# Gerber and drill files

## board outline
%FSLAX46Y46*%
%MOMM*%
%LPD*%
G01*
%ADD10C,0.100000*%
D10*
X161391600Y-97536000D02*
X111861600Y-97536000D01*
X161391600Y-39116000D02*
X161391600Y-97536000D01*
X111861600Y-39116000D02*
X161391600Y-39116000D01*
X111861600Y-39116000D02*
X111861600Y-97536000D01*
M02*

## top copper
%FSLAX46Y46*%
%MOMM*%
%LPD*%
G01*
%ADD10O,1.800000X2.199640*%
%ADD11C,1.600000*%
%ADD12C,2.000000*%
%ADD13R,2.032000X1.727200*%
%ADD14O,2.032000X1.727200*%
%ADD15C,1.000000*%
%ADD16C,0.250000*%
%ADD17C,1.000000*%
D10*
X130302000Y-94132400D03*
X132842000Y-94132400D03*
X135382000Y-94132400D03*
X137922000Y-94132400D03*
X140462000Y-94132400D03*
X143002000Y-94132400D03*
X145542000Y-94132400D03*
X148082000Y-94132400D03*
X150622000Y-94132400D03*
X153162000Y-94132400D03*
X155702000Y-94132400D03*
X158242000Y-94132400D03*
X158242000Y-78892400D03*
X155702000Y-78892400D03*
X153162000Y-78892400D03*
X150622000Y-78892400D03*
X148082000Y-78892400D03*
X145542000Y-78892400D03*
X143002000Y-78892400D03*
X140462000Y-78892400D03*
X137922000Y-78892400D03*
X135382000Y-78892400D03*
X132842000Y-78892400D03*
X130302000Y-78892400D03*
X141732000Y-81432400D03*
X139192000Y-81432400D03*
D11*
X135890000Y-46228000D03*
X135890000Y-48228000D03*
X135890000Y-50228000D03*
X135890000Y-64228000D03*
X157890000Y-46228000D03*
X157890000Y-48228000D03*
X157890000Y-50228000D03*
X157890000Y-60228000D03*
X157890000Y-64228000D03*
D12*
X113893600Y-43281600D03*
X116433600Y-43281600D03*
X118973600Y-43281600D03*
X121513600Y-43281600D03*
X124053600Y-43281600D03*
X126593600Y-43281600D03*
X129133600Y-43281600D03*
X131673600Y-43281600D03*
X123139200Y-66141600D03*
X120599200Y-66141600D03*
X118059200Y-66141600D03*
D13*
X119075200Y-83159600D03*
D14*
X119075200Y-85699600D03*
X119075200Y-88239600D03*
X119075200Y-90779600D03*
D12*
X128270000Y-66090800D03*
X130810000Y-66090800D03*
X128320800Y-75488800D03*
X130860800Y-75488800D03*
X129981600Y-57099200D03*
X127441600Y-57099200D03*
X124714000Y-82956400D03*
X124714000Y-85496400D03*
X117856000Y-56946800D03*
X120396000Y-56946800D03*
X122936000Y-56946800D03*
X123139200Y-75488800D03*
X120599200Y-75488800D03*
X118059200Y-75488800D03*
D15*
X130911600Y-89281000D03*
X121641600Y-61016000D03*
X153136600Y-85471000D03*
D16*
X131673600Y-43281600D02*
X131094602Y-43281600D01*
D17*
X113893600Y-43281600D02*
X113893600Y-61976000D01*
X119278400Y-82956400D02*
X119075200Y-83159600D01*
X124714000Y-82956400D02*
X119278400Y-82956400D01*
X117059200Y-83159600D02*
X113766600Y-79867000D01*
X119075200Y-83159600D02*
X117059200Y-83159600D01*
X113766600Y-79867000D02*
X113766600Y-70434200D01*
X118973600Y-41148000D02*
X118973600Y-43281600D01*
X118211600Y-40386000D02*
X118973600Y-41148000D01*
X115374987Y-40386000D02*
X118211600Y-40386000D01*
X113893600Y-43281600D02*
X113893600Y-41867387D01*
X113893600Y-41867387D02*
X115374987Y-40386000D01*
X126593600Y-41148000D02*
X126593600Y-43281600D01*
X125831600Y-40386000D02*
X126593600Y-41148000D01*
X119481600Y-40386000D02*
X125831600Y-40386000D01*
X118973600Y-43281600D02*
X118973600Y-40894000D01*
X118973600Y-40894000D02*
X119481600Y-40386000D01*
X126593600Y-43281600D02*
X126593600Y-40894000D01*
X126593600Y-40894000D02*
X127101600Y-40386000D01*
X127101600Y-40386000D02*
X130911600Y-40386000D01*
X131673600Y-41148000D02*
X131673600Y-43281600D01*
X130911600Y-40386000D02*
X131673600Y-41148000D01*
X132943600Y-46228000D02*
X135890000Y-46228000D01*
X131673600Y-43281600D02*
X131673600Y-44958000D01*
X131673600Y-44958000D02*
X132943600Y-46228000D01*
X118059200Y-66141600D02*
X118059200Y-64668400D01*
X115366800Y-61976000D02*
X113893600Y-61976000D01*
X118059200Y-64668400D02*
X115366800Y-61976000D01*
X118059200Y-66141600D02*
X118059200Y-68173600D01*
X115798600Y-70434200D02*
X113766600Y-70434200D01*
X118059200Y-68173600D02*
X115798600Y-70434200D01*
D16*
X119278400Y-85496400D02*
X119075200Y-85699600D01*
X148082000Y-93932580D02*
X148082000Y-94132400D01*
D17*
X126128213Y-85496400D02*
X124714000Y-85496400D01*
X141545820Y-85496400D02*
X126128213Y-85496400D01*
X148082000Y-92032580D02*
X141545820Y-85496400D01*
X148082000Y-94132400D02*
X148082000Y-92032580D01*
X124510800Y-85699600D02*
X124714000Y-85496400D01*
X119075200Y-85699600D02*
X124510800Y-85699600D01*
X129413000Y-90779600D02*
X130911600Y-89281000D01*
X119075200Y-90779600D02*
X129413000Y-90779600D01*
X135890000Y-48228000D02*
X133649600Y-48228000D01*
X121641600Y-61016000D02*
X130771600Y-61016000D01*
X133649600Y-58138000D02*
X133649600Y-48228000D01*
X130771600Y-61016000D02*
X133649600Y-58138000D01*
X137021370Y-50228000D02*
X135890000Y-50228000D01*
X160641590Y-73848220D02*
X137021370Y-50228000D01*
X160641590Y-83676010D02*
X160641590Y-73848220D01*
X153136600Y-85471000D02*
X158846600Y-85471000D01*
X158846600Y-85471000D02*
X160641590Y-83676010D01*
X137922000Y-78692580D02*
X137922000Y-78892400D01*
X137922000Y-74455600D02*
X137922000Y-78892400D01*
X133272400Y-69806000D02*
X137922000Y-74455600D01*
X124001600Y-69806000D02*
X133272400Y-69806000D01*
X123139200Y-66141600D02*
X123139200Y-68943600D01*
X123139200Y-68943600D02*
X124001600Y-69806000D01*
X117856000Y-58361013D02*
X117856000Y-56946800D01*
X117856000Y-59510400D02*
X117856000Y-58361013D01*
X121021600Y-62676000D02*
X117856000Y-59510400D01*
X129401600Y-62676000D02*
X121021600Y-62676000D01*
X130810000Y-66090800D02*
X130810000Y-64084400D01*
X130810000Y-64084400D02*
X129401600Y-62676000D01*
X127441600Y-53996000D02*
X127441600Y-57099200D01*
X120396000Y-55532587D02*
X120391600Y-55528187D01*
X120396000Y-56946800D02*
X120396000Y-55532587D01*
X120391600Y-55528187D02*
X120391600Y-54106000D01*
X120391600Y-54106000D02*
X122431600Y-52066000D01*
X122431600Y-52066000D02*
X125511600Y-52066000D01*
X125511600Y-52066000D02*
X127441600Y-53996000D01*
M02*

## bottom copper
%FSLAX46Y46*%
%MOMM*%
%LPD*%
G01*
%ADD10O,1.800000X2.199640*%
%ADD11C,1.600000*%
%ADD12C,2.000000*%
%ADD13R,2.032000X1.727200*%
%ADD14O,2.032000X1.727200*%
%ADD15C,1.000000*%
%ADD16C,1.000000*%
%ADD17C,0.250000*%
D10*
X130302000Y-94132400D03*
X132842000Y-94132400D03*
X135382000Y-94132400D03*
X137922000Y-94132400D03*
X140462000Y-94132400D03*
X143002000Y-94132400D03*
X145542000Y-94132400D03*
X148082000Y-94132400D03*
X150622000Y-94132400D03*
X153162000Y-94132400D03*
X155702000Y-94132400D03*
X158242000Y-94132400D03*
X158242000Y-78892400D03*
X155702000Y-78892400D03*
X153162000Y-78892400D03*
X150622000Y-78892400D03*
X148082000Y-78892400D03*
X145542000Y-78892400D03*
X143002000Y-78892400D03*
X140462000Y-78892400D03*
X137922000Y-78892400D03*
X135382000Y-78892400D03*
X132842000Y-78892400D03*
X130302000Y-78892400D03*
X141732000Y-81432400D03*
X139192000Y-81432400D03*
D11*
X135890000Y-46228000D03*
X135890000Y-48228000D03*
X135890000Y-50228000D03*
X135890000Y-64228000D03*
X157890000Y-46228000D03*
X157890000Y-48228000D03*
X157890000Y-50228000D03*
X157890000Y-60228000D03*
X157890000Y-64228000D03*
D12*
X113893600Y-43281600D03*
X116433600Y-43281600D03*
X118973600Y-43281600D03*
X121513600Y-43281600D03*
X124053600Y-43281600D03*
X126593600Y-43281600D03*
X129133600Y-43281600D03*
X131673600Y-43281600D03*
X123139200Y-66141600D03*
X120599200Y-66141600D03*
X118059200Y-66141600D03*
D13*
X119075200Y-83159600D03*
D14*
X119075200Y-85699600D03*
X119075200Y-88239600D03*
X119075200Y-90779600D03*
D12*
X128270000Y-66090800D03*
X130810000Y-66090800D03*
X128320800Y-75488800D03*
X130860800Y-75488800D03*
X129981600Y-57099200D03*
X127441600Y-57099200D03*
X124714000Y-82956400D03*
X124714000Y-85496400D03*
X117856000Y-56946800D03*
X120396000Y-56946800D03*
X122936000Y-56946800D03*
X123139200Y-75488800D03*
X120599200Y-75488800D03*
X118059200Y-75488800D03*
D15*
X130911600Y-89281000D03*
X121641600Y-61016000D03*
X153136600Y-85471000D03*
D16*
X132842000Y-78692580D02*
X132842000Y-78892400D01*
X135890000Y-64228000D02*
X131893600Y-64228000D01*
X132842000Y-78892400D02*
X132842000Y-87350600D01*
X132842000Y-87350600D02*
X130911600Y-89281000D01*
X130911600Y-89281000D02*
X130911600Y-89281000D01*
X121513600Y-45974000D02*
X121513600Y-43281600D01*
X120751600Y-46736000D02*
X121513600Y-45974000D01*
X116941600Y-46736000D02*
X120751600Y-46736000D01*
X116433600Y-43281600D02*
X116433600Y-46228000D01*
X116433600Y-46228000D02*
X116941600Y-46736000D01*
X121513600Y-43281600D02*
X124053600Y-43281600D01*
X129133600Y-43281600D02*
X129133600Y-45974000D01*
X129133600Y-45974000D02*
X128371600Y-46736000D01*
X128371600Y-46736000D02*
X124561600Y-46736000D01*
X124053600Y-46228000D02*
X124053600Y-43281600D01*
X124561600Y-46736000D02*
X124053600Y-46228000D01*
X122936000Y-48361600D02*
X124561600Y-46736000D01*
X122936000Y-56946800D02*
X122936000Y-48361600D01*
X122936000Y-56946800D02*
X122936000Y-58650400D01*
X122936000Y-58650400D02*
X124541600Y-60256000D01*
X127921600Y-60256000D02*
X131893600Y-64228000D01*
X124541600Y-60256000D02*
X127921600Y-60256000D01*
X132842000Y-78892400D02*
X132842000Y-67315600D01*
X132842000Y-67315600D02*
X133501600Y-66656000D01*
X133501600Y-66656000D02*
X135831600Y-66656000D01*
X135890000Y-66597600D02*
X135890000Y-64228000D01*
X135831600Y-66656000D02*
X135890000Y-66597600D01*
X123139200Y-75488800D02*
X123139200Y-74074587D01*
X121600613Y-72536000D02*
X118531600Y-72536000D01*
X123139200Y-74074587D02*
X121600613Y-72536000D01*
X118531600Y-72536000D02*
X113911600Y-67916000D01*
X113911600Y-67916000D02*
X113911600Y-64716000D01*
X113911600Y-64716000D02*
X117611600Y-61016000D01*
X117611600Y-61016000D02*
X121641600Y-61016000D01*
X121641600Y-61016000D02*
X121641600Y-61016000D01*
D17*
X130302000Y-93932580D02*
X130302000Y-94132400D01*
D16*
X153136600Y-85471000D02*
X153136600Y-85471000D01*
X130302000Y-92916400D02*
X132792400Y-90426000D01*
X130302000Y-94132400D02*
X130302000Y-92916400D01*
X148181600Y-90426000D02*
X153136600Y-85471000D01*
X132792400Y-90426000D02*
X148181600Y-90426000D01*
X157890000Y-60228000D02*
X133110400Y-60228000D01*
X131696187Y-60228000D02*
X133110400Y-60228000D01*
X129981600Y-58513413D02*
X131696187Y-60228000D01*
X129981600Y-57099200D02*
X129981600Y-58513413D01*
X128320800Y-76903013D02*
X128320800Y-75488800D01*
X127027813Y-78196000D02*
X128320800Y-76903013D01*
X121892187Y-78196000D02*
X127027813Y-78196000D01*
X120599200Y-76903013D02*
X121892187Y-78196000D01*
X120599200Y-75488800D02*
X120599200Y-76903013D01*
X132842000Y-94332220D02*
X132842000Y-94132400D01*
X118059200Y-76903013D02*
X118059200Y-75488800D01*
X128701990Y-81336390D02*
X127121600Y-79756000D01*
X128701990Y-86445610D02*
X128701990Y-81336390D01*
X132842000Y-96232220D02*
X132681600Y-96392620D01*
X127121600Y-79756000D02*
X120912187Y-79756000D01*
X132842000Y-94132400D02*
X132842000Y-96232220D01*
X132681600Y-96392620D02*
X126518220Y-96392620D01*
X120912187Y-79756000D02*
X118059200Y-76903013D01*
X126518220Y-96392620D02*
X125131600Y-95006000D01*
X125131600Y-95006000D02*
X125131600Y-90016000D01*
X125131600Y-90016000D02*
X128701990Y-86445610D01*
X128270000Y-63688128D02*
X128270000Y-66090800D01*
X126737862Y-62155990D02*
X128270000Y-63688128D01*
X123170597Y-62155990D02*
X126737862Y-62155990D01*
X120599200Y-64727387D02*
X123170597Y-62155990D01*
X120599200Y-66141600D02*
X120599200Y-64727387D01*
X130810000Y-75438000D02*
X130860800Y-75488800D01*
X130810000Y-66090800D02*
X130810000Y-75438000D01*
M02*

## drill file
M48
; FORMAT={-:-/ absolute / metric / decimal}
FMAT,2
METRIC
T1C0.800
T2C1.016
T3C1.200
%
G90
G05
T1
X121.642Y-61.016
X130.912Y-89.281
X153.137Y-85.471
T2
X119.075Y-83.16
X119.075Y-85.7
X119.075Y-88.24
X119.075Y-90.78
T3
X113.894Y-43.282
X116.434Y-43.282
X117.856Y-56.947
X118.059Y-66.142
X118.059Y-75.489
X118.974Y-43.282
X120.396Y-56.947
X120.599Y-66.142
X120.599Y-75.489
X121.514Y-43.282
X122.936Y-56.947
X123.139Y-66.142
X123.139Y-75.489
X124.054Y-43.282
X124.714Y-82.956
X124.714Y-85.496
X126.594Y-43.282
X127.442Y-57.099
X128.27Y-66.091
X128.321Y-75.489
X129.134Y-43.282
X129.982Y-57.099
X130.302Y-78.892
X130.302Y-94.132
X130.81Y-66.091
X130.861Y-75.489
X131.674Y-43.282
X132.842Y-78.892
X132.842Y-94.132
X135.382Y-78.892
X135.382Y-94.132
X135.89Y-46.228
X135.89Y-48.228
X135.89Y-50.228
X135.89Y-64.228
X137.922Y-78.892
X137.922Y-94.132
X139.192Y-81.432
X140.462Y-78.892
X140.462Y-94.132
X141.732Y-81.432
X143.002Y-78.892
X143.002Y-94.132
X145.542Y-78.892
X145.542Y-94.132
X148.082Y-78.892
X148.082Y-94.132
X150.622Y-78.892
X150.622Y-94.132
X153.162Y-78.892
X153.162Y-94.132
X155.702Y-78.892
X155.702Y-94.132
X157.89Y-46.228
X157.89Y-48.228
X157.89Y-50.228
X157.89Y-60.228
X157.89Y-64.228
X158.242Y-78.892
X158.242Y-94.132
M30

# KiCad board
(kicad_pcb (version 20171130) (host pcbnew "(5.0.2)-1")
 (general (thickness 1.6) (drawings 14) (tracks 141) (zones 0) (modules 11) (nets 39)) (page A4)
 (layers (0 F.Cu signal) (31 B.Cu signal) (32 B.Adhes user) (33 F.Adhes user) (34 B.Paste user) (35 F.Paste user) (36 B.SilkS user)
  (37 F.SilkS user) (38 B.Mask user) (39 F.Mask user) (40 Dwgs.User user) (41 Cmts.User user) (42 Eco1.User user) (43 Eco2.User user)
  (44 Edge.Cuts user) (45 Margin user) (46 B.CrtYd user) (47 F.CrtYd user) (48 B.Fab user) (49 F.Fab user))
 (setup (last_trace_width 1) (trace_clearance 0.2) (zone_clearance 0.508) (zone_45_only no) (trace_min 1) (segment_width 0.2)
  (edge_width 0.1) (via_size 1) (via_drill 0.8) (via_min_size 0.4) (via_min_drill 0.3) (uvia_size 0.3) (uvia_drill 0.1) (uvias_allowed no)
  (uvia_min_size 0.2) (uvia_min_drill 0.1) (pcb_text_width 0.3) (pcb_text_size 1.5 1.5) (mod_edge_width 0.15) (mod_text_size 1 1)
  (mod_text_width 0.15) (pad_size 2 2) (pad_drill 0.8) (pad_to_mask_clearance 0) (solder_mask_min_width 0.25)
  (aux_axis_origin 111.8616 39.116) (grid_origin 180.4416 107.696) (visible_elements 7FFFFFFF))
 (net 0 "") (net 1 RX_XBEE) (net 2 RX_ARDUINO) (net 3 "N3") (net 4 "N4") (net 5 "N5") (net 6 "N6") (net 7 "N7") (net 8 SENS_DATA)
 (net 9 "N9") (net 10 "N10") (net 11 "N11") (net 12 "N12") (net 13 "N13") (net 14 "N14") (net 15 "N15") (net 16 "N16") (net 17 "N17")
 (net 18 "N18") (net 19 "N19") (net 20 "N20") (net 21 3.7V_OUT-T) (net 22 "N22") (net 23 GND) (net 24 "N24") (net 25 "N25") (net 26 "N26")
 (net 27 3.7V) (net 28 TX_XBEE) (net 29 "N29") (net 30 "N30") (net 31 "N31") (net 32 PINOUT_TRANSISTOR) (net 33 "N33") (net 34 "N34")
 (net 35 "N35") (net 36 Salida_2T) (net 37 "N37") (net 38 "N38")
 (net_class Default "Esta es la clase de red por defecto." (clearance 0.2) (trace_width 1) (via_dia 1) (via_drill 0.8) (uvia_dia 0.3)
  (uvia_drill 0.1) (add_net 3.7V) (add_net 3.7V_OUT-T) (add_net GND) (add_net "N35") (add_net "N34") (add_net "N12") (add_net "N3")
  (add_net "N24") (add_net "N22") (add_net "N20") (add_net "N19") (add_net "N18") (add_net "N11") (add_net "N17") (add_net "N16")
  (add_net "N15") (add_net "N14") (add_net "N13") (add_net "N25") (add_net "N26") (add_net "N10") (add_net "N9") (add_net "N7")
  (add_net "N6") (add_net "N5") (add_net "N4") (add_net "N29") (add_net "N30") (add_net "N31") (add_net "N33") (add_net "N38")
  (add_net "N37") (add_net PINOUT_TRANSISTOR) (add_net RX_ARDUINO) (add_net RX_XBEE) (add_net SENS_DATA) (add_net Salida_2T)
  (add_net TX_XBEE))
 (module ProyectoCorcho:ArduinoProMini (layer F.Cu) (at 144.272 86.5124)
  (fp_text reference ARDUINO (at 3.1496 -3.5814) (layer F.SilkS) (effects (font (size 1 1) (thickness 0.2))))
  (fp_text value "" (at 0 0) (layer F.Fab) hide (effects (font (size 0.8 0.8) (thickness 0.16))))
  (pad 12 thru_hole oval (at -13.97 7.62) (size 1.8 2.19964) (drill 1.2) (layers *.Cu *.Mask) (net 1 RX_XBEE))
  (pad 11 thru_hole oval (at -11.43 7.62) (size 1.8 2.19964) (drill 1.2) (layers *.Cu *.Mask) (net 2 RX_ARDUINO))
  (pad 10 thru_hole oval (at -8.89 7.62) (size 1.8 2.19964) (drill 1.2) (layers *.Cu *.Mask) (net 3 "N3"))
  (pad 9 thru_hole oval (at -6.35 7.62) (size 1.8 2.19964) (drill 1.2) (layers *.Cu *.Mask) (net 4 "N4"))
  (pad 8 thru_hole oval (at -3.81 7.62) (size 1.8 2.19964) (drill 1.2) (layers *.Cu *.Mask) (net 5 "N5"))
  (pad 7 thru_hole oval (at -1.27 7.62) (size 1.8 2.19964) (drill 1.2) (layers *.Cu *.Mask) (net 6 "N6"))
  (pad 6 thru_hole oval (at 1.27 7.62) (size 1.8 2.19964) (drill 1.2) (layers *.Cu *.Mask) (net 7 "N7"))
  (pad 5 thru_hole oval (at 3.81 7.62) (size 1.8 2.19964) (drill 1.2) (layers *.Cu *.Mask) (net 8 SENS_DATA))
  (pad 4 thru_hole oval (at 6.35 7.62) (size 1.8 2.19964) (drill 1.2) (layers *.Cu *.Mask) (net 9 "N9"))
  (pad 3 thru_hole oval (at 8.89 7.62) (size 1.8 2.19964) (drill 1.2) (layers *.Cu *.Mask) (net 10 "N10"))
  (pad 2 thru_hole oval (at 11.43 7.62) (size 1.8 2.19964) (drill 1.2) (layers *.Cu *.Mask) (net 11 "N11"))
  (pad 1 thru_hole oval (at 13.97 7.62) (size 1.8 2.19964) (drill 1.2) (layers *.Cu *.Mask) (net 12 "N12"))
  (pad 24 thru_hole oval (at 13.97 -7.62) (size 1.8 2.19964) (drill 1.2) (layers *.Cu *.Mask) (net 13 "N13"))
  (pad 23 thru_hole oval (at 11.43 -7.62) (size 1.8 2.19964) (drill 1.2) (layers *.Cu *.Mask) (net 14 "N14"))
  (pad 22 thru_hole oval (at 8.89 -7.62) (size 1.8 2.19964) (drill 1.2) (layers *.Cu *.Mask) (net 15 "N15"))
  (pad 21 thru_hole oval (at 6.35 -7.62) (size 1.8 2.19964) (drill 1.2) (layers *.Cu *.Mask) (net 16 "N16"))
  (pad 20 thru_hole oval (at 3.81 -7.62) (size 1.8 2.19964) (drill 1.2) (layers *.Cu *.Mask) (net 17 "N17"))
  (pad 19 thru_hole oval (at 1.27 -7.62) (size 1.8 2.19964) (drill 1.2) (layers *.Cu *.Mask) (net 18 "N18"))
  (pad 18 thru_hole oval (at -1.27 -7.62) (size 1.8 2.19964) (drill 1.2) (layers *.Cu *.Mask) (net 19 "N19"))
  (pad 17 thru_hole oval (at -3.81 -7.62) (size 1.8 2.19964) (drill 1.2) (layers *.Cu *.Mask) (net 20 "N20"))
  (pad 16 thru_hole oval (at -6.35 -7.62) (size 1.8 2.19964) (drill 1.2) (layers *.Cu *.Mask) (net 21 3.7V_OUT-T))
  (pad 15 thru_hole oval (at -8.89 -7.62) (size 1.8 2.19964) (drill 1.2) (layers *.Cu *.Mask) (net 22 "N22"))
  (pad 14 thru_hole oval (at -11.43 -7.62) (size 1.8 2.19964) (drill 1.2) (layers *.Cu *.Mask) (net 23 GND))
  (pad 13 thru_hole oval (at -13.97 -7.62) (size 1.8 2.19964) (drill 1.2) (layers *.Cu *.Mask) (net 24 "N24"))
  (pad 25 thru_hole oval (at -2.54 -5.08) (size 1.8 2.19964) (drill 1.2) (layers *.Cu *.Mask) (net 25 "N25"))
  (pad 26 thru_hole oval (at -5.08 -5.08) (size 1.8 2.19964) (drill 1.2) (layers *.Cu *.Mask) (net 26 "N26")))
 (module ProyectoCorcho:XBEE (layer F.Cu) (at 134.62 44.958)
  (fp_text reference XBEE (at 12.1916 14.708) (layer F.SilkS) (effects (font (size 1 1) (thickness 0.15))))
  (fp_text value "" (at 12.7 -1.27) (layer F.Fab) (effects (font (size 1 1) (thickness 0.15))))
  (pad 1 thru_hole circle (at 1.27 1.27) (size 1.6 1.6) (drill 1.2) (layers *.Cu *.Mask) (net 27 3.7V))
  (pad 2 thru_hole circle (at 1.27 3.27) (size 1.6 1.6) (drill 1.2) (layers *.Cu *.Mask) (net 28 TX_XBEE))
  (pad 3 thru_hole circle (at 1.27 5.27) (size 1.6 1.6) (drill 1.2) (layers *.Cu *.Mask) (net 1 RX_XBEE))
  (pad 4 thru_hole circle (at 1.27 19.27) (size 1.6 1.6) (drill 1.2) (layers *.Cu *.Mask) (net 23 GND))
  (pad 5 thru_hole circle (at 23.27 1.27) (size 1.6 1.6) (drill 1.2) (layers *.Cu *.Mask) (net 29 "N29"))
  (pad 6 thru_hole circle (at 23.27 3.27) (size 1.6 1.6) (drill 1.2) (layers *.Cu *.Mask) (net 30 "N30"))
  (pad 7 thru_hole circle (at 23.27 5.27) (size 1.6 1.6) (drill 1.2) (layers *.Cu *.Mask) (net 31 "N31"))
  (pad 8 thru_hole circle (at 23.27 15.27) (size 1.6 1.6) (drill 1.2) (layers *.Cu *.Mask) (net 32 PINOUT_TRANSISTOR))
  (pad 9 thru_hole circle (at 23.27 19.27) (size 1.6 1.6) (drill 1.2) (layers *.Cu *.Mask) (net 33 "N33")))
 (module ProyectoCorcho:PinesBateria (layer F.Cu) (at 112.6236 42.0116)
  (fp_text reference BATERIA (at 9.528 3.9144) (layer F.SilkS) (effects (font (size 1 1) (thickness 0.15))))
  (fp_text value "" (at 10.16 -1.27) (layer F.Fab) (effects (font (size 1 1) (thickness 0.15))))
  (pad 1 thru_hole circle (at 1.27 1.27) (size 2 2) (drill 1.2) (layers *.Cu *.Mask) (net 27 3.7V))
  (pad 2 thru_hole circle (at 3.81 1.27) (size 2 2) (drill 1.2) (layers *.Cu *.Mask) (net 23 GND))
  (pad 3 thru_hole circle (at 6.35 1.27) (size 2 2) (drill 1.2) (layers *.Cu *.Mask) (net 27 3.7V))
  (pad 4 thru_hole circle (at 8.89 1.27) (size 2 2) (drill 1.2) (layers *.Cu *.Mask) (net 23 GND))
  (pad 5 thru_hole circle (at 11.43 1.27) (size 2 2) (drill 1.2) (layers *.Cu *.Mask) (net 23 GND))
  (pad 6 thru_hole circle (at 13.97 1.27) (size 2 2) (drill 1.2) (layers *.Cu *.Mask) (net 27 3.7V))
  (pad 7 thru_hole circle (at 16.51 1.27) (size 2 2) (drill 1.2) (layers *.Cu *.Mask) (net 23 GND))
  (pad 8 thru_hole circle (at 19.05 1.27) (size 2 2) (drill 1.2) (layers *.Cu *.Mask) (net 27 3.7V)))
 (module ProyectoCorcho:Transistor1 (layer B.Cu) (at 120.5992 66.1416)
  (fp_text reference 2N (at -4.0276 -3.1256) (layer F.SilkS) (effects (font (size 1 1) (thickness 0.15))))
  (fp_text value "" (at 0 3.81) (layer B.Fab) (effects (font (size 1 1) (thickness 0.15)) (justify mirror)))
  (pad 3 thru_hole circle (at 2.54 0) (size 2 2) (drill 1.2) (layers *.Cu *.Mask) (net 21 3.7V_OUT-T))
  (pad 2 thru_hole circle (at 0 0) (size 2 2) (drill 1.2) (layers *.Cu *.Mask) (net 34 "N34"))
  (pad 1 thru_hole circle (at -2.54 0) (size 2 2) (drill 1.2) (layers *.Cu *.Mask) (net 27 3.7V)))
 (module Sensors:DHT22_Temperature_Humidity (layer F.Cu) (at 119.0752 86.9696 270)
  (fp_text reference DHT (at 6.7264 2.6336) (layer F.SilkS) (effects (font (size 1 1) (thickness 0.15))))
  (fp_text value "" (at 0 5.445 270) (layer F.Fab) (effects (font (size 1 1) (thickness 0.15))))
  (pad 1 thru_hole rect (at -3.81 0) (size 2.032 1.7272) (drill 1.016) (layers *.Cu *.Mask F.SilkS) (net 27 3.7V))
  (pad 2 thru_hole oval (at -1.27 0) (size 2.032 1.7272) (drill 1.016) (layers *.Cu *.Mask F.SilkS) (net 8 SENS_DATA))
  (pad 3 thru_hole oval (at 1.27 0) (size 2.032 1.7272) (drill 1.016) (layers *.Cu *.Mask F.SilkS) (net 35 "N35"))
  (pad 4 thru_hole oval (at 3.81 0) (size 2.032 1.7272) (drill 1.016) (layers *.Cu *.Mask F.SilkS) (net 23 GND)))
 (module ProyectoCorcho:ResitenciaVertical (layer F.Cu) (at 128.27 66.0908)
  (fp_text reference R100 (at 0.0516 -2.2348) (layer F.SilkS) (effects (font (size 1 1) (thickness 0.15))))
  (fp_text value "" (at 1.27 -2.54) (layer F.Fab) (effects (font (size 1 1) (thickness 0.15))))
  (pad 1 thru_hole circle (at 0 0) (size 2 2) (drill 1.2) (layers *.Cu *.Mask) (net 34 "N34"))
  (pad 2 thru_hole circle (at 2.54 0) (size 2 2) (drill 1.2) (layers *.Cu *.Mask) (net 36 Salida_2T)))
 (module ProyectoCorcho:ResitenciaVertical (layer F.Cu) (at 128.3208 75.4888)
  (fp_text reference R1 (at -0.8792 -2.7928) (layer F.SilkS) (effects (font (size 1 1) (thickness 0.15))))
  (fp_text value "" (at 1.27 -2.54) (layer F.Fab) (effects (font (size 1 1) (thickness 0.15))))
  (pad 1 thru_hole circle (at 0 0) (size 2 2) (drill 1.2) (layers *.Cu *.Mask) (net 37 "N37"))
  (pad 2 thru_hole circle (at 2.54 0) (size 2 2) (drill 1.2) (layers *.Cu *.Mask) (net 36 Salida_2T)))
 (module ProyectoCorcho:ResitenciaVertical (layer F.Cu) (at 127.4416 57.0992)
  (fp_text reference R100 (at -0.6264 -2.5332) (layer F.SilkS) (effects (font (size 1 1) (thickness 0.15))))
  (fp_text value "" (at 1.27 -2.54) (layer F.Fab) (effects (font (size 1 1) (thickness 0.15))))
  (pad 2 thru_hole circle (at 2.54 0) (size 2 2) (drill 1.2) (layers *.Cu *.Mask) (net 32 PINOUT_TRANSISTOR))
  (pad 1 thru_hole circle (at 0 0) (size 2 2) (drill 1.2) (layers *.Cu *.Mask) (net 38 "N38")))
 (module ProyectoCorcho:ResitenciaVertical (layer F.Cu) (at 124.714 82.9564 270)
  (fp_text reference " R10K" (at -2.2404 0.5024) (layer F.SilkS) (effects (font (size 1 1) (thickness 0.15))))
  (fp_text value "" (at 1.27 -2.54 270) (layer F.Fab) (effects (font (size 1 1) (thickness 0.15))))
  (pad 1 thru_hole circle (at 0 0 270) (size 2 2) (drill 1.2) (layers *.Cu *.Mask) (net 27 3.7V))
  (pad 2 thru_hole circle (at 2.54 0 270) (size 2 2) (drill 1.2) (layers *.Cu *.Mask) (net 8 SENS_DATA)))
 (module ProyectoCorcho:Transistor (layer F.Cu) (at 120.396 56.9468)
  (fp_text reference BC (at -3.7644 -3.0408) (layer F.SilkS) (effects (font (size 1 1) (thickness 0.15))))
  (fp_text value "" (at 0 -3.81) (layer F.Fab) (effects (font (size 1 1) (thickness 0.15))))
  (pad 1 thru_hole circle (at -2.54 0) (size 2 2) (drill 1.2) (layers *.Cu *.Mask) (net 36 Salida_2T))
  (pad 2 thru_hole circle (at 0 0) (size 2 2) (drill 1.2) (layers *.Cu *.Mask) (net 38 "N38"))
  (pad 3 thru_hole circle (at 2.54 0) (size 2 2) (drill 1.2) (layers *.Cu *.Mask) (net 23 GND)))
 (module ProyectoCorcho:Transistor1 (layer B.Cu) (at 120.5992 75.4888 180)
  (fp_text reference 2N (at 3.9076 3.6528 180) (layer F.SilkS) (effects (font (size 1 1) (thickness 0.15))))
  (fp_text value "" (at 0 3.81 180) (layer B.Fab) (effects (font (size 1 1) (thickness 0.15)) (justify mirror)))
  (pad 1 thru_hole circle (at -2.54 0 180) (size 2 2) (drill 1.2) (layers *.Cu *.Mask) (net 28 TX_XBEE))
  (pad 2 thru_hole circle (at 0 0 180) (size 2 2) (drill 1.2) (layers *.Cu *.Mask) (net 37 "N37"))
  (pad 3 thru_hole circle (at 2.54 0 180) (size 2 2) (drill 1.2) (layers *.Cu *.Mask) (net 2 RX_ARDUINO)))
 (gr_line (start 161.3916 97.536) (end 111.8616 97.536) (layer Edge.Cuts) (width 0.1))
 (gr_line (start 161.3916 39.116) (end 161.3916 97.536) (layer Edge.Cuts) (width 0.1))
 (gr_line (start 111.8616 39.116) (end 161.3916 39.116) (layer Edge.Cuts) (width 0.1))
 (gr_line (start 111.8616 39.116) (end 111.8616 97.536) (layer Edge.Cuts) (width 0.1))
 (segment (start 131.6736 43.2816) (end 131.094602 43.2816) (width 0.25) (layer F.Cu) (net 27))
 (segment (start 113.8936 43.2816) (end 113.8936 61.976) (width 1) (layer F.Cu) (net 27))
 (segment (start 119.2784 82.9564) (end 119.0752 83.1596) (width 1) (layer F.Cu) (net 27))
 (segment (start 124.714 82.9564) (end 119.2784 82.9564) (width 1) (layer F.Cu) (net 27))
 (segment (start 117.0592 83.1596) (end 113.7666 79.867) (width 1) (layer F.Cu) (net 27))
 (segment (start 119.0752 83.1596) (end 117.0592 83.1596) (width 1) (layer F.Cu) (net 27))
 (segment (start 113.7666 79.867) (end 113.7666 70.4342) (width 1) (layer F.Cu) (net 27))
 (segment (start 118.9736 41.148) (end 118.9736 43.2816) (width 1) (layer F.Cu) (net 27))
 (segment (start 118.2116 40.386) (end 118.9736 41.148) (width 1) (layer F.Cu) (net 27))
 (segment (start 115.374987 40.386) (end 118.2116 40.386) (width 1) (layer F.Cu) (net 27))
 (segment (start 113.8936 43.2816) (end 113.8936 41.867387) (width 1) (layer F.Cu) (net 27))
 (segment (start 113.8936 41.867387) (end 115.374987 40.386) (width 1) (layer F.Cu) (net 27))
 (segment (start 126.5936 41.148) (end 126.5936 43.2816) (width 1) (layer F.Cu) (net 27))
 (segment (start 125.8316 40.386) (end 126.5936 41.148) (width 1) (layer F.Cu) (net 27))
 (segment (start 119.4816 40.386) (end 125.8316 40.386) (width 1) (layer F.Cu) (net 27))
 (segment (start 118.9736 43.2816) (end 118.9736 40.894) (width 1) (layer F.Cu) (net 27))
 (segment (start 118.9736 40.894) (end 119.4816 40.386) (width 1) (layer F.Cu) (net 27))
 (segment (start 126.5936 43.2816) (end 126.5936 40.894) (width 1) (layer F.Cu) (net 27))
 (segment (start 126.5936 40.894) (end 127.1016 40.386) (width 1) (layer F.Cu) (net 27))
 (segment (start 127.1016 40.386) (end 130.9116 40.386) (width 1) (layer F.Cu) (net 27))
 (segment (start 131.6736 41.148) (end 131.6736 43.2816) (width 1) (layer F.Cu) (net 27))
 (segment (start 130.9116 40.386) (end 131.6736 41.148) (width 1) (layer F.Cu) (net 27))
 (segment (start 132.9436 46.228) (end 135.89 46.228) (width 1) (layer F.Cu) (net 27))
 (segment (start 131.6736 43.2816) (end 131.6736 44.958) (width 1) (layer F.Cu) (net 27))
 (segment (start 131.6736 44.958) (end 132.9436 46.228) (width 1) (layer F.Cu) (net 27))
 (segment (start 118.0592 66.1416) (end 118.0592 64.6684) (width 1) (layer F.Cu) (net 27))
 (segment (start 115.3668 61.976) (end 113.8936 61.976) (width 1) (layer F.Cu) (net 27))
 (segment (start 118.0592 64.6684) (end 115.3668 61.976) (width 1) (layer F.Cu) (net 27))
 (segment (start 118.0592 66.1416) (end 118.0592 68.1736) (width 1) (layer F.Cu) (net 27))
 (segment (start 115.7986 70.4342) (end 113.7666 70.4342) (width 1) (layer F.Cu) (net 27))
 (segment (start 118.0592 68.1736) (end 115.7986 70.4342) (width 1) (layer F.Cu) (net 27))
 (segment (start 119.2784 85.4964) (end 119.0752 85.6996) (width 0.25) (layer F.Cu) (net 8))
 (segment (start 148.082 93.93258) (end 148.082 94.1324) (width 0.25) (layer F.Cu) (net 8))
 (segment (start 126.128213 85.4964) (end 124.714 85.4964) (width 1) (layer F.Cu) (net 8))
 (segment (start 141.54582 85.4964) (end 126.128213 85.4964) (width 1) (layer F.Cu) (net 8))
 (segment (start 148.082 92.03258) (end 141.54582 85.4964) (width 1) (layer F.Cu) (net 8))
 (segment (start 148.082 94.1324) (end 148.082 92.03258) (width 1) (layer F.Cu) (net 8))
 (segment (start 124.5108 85.6996) (end 124.714 85.4964) (width 1) (layer F.Cu) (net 8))
 (segment (start 119.0752 85.6996) (end 124.5108 85.6996) (width 1) (layer F.Cu) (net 8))
 (segment (start 132.842 78.69258) (end 132.842 78.8924) (width 1) (layer B.Cu) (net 23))
 (segment (start 135.89 64.228) (end 131.8936 64.228) (width 1) (layer B.Cu) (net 23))
 (segment (start 132.842 78.8924) (end 132.842 87.3506) (width 1) (layer B.Cu) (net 23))
 (segment (start 132.842 87.3506) (end 130.9116 89.281) (width 1) (layer B.Cu) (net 23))
 (segment (start 130.9116 89.281) (end 130.9116 89.281) (width 1) (layer B.Cu) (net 23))
 (via (at 130.9116 89.281) (size 1) (drill 0.8) (layers F.Cu B.Cu) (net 23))
 (segment (start 129.413 90.7796) (end 130.9116 89.281) (width 1) (layer F.Cu) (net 23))
 (segment (start 119.0752 90.7796) (end 129.413 90.7796) (width 1) (layer F.Cu) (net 23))
 (segment (start 121.5136 45.974) (end 121.5136 43.2816) (width 1) (layer B.Cu) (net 23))
 (segment (start 120.7516 46.736) (end 121.5136 45.974) (width 1) (layer B.Cu) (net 23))
 (segment (start 116.9416 46.736) (end 120.7516 46.736) (width 1) (layer B.Cu) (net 23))
 (segment (start 116.4336 43.2816) (end 116.4336 46.228) (width 1) (layer B.Cu) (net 23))
 (segment (start 116.4336 46.228) (end 116.9416 46.736) (width 1) (layer B.Cu) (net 23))
 (segment (start 121.5136 43.2816) (end 124.0536 43.2816) (width 1) (layer B.Cu) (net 23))
 (segment (start 129.1336 43.2816) (end 129.1336 45.974) (width 1) (layer B.Cu) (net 23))
 (segment (start 129.1336 45.974) (end 128.3716 46.736) (width 1) (layer B.Cu) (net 23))
 (segment (start 128.3716 46.736) (end 124.5616 46.736) (width 1) (layer B.Cu) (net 23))
 (segment (start 124.0536 46.228) (end 124.0536 43.2816) (width 1) (layer B.Cu) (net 23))
 (segment (start 124.5616 46.736) (end 124.0536 46.228) (width 1) (layer B.Cu) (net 23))
 (segment (start 122.936 48.3616) (end 124.5616 46.736) (width 1) (layer B.Cu) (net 23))
 (segment (start 122.936 56.9468) (end 122.936 48.3616) (width 1) (layer B.Cu) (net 23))
 (segment (start 122.936 56.9468) (end 122.936 58.6504) (width 1) (layer B.Cu) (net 23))
 (segment (start 122.936 58.6504) (end 124.5416 60.256) (width 1) (layer B.Cu) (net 23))
 (segment (start 127.9216 60.256) (end 131.8936 64.228) (width 1) (layer B.Cu) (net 23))
 (segment (start 124.5416 60.256) (end 127.9216 60.256) (width 1) (layer B.Cu) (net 23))
 (segment (start 132.842 78.8924) (end 132.842 67.3156) (width 1) (layer B.Cu) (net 23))
 (segment (start 132.842 67.3156) (end 133.5016 66.656) (width 1) (layer B.Cu) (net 23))
 (segment (start 133.5016 66.656) (end 135.8316 66.656) (width 1) (layer B.Cu) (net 23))
 (segment (start 135.89 66.5976) (end 135.89 64.228) (width 1) (layer B.Cu) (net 23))
 (segment (start 135.8316 66.656) (end 135.89 66.5976) (width 1) (layer B.Cu) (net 23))
 (segment (start 123.1392 75.4888) (end 123.1392 74.074587) (width 1) (layer B.Cu) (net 28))
 (segment (start 135.89 48.228) (end 133.6496 48.228) (width 1) (layer F.Cu) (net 28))
 (segment (start 121.600613 72.536) (end 118.5316 72.536) (width 1) (layer B.Cu) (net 28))
 (segment (start 123.1392 74.074587) (end 121.600613 72.536) (width 1) (layer B.Cu) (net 28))
 (segment (start 118.5316 72.536) (end 113.9116 67.916) (width 1) (layer B.Cu) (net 28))
 (segment (start 113.9116 67.916) (end 113.9116 64.716) (width 1) (layer B.Cu) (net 28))
 (segment (start 113.9116 64.716) (end 117.6116 61.016) (width 1) (layer B.Cu) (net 28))
 (segment (start 117.6116 61.016) (end 121.6416 61.016) (width 1) (layer B.Cu) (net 28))
 (segment (start 121.6416 61.016) (end 121.6416 61.016) (width 1) (layer B.Cu) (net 28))
 (via (at 121.6416 61.016) (size 1) (drill 0.8) (layers F.Cu B.Cu) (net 28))
 (segment (start 121.6416 61.016) (end 130.7716 61.016) (width 1) (layer F.Cu) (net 28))
 (segment (start 133.6496 58.138) (end 133.6496 48.228) (width 1) (layer F.Cu) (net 28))
 (segment (start 130.7716 61.016) (end 133.6496 58.138) (width 1) (layer F.Cu) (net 28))
 (segment (start 130.302 93.93258) (end 130.302 94.1324) (width 0.25) (layer B.Cu) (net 1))
 (segment (start 153.1366 85.471) (end 153.1366 85.471) (width 1) (layer B.Cu) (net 1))
 (via (at 153.1366 85.471) (size 1) (drill 0.8) (layers F.Cu B.Cu) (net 1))
 (segment (start 130.302 92.9164) (end 132.7924 90.426) (width 1) (layer B.Cu) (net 1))
 (segment (start 130.302 94.1324) (end 130.302 92.9164) (width 1) (layer B.Cu) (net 1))
 (segment (start 148.1816 90.426) (end 153.1366 85.471) (width 1) (layer B.Cu) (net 1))
 (segment (start 132.7924 90.426) (end 148.1816 90.426) (width 1) (layer B.Cu) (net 1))
 (segment (start 137.02137 50.228) (end 135.89 50.228) (width 1) (layer F.Cu) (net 1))
 (segment (start 160.64159 73.84822) (end 137.02137 50.228) (width 1) (layer F.Cu) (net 1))
 (segment (start 160.64159 83.67601) (end 160.64159 73.84822) (width 1) (layer F.Cu) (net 1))
 (segment (start 153.1366 85.471) (end 158.8466 85.471) (width 1) (layer F.Cu) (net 1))
 (segment (start 158.8466 85.471) (end 160.64159 83.67601) (width 1) (layer F.Cu) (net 1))
 (segment (start 157.89 60.228) (end 133.1104 60.228) (width 1) (layer B.Cu) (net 32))
 (segment (start 131.696187 60.228) (end 133.1104 60.228) (width 1) (layer B.Cu) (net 32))
 (segment (start 129.9816 58.513413) (end 131.696187 60.228) (width 1) (layer B.Cu) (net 32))
 (segment (start 129.9816 57.0992) (end 129.9816 58.513413) (width 1) (layer B.Cu) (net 32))
 (segment (start 128.3208 76.903013) (end 128.3208 75.4888) (width 1) (layer B.Cu) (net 37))
 (segment (start 127.027813 78.196) (end 128.3208 76.903013) (width 1) (layer B.Cu) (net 37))
 (segment (start 121.892187 78.196) (end 127.027813 78.196) (width 1) (layer B.Cu) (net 37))
 (segment (start 120.5992 76.903013) (end 121.892187 78.196) (width 1) (layer B.Cu) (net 37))
 (segment (start 120.5992 75.4888) (end 120.5992 76.903013) (width 1) (layer B.Cu) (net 37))
 (segment (start 132.842 94.33222) (end 132.842 94.1324) (width 1) (layer B.Cu) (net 2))
 (segment (start 118.0592 76.903013) (end 118.0592 75.4888) (width 1) (layer B.Cu) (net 2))
 (segment (start 128.70199 81.33639) (end 127.1216 79.756) (width 1) (layer B.Cu) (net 2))
 (segment (start 128.70199 86.44561) (end 128.70199 81.33639) (width 1) (layer B.Cu) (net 2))
 (segment (start 132.842 96.23222) (end 132.6816 96.39262) (width 1) (layer B.Cu) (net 2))
 (segment (start 127.1216 79.756) (end 120.912187 79.756) (width 1) (layer B.Cu) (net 2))
 (segment (start 132.842 94.1324) (end 132.842 96.23222) (width 1) (layer B.Cu) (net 2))
 (segment (start 132.6816 96.39262) (end 126.51822 96.39262) (width 1) (layer B.Cu) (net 2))
 (segment (start 120.912187 79.756) (end 118.0592 76.903013) (width 1) (layer B.Cu) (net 2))
 (segment (start 126.51822 96.39262) (end 125.1316 95.006) (width 1) (layer B.Cu) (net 2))
 (segment (start 125.1316 95.006) (end 125.1316 90.016) (width 1) (layer B.Cu) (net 2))
 (segment (start 125.1316 90.016) (end 128.70199 86.44561) (width 1) (layer B.Cu) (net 2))
 (segment (start 137.922 78.69258) (end 137.922 78.8924) (width 1) (layer F.Cu) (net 21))
 (segment (start 137.922 74.4556) (end 137.922 78.8924) (width 1) (layer F.Cu) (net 21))
 (segment (start 133.2724 69.806) (end 137.922 74.4556) (width 1) (layer F.Cu) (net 21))
 (segment (start 124.0016 69.806) (end 133.2724 69.806) (width 1) (layer F.Cu) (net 21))
 (segment (start 123.1392 66.1416) (end 123.1392 68.9436) (width 1) (layer F.Cu) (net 21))
 (segment (start 123.1392 68.9436) (end 124.0016 69.806) (width 1) (layer F.Cu) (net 21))
 (segment (start 128.27 63.688128) (end 128.27 66.0908) (width 1) (layer B.Cu) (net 34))
 (segment (start 126.737862 62.15599) (end 128.27 63.688128) (width 1) (layer B.Cu) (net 34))
 (segment (start 123.170597 62.15599) (end 126.737862 62.15599) (width 1) (layer B.Cu) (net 34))
 (segment (start 120.5992 64.727387) (end 123.170597 62.15599) (width 1) (layer B.Cu) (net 34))
 (segment (start 120.5992 66.1416) (end 120.5992 64.727387) (width 1) (layer B.Cu) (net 34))
 (segment (start 130.81 75.438) (end 130.8608 75.4888) (width 1) (layer B.Cu) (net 36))
 (segment (start 130.81 66.0908) (end 130.81 75.438) (width 1) (layer B.Cu) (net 36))
 (segment (start 117.856 58.361013) (end 117.856 56.9468) (width 1) (layer F.Cu) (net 36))
 (segment (start 117.856 59.5104) (end 117.856 58.361013) (width 1) (layer F.Cu) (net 36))
 (segment (start 121.0216 62.676) (end 117.856 59.5104) (width 1) (layer F.Cu) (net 36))
 (segment (start 129.4016 62.676) (end 121.0216 62.676) (width 1) (layer F.Cu) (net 36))
 (segment (start 130.81 66.0908) (end 130.81 64.0844) (width 1) (layer F.Cu) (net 36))
 (segment (start 130.81 64.0844) (end 129.4016 62.676) (width 1) (layer F.Cu) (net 36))
 (segment (start 127.4416 53.996) (end 127.4416 57.0992) (width 1) (layer F.Cu) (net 38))
 (segment (start 120.396 55.532587) (end 120.3916 55.528187) (width 1) (layer F.Cu) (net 38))
 (segment (start 120.396 56.9468) (end 120.396 55.532587) (width 1) (layer F.Cu) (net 38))
 (segment (start 120.3916 55.528187) (end 120.3916 54.106) (width 1) (layer F.Cu) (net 38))
 (segment (start 120.3916 54.106) (end 122.4316 52.066) (width 1) (layer F.Cu) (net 38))
 (segment (start 122.4316 52.066) (end 125.5116 52.066) (width 1) (layer F.Cu) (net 38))
 (segment (start 125.5116 52.066) (end 127.4416 53.996) (width 1) (layer F.Cu) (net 38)))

